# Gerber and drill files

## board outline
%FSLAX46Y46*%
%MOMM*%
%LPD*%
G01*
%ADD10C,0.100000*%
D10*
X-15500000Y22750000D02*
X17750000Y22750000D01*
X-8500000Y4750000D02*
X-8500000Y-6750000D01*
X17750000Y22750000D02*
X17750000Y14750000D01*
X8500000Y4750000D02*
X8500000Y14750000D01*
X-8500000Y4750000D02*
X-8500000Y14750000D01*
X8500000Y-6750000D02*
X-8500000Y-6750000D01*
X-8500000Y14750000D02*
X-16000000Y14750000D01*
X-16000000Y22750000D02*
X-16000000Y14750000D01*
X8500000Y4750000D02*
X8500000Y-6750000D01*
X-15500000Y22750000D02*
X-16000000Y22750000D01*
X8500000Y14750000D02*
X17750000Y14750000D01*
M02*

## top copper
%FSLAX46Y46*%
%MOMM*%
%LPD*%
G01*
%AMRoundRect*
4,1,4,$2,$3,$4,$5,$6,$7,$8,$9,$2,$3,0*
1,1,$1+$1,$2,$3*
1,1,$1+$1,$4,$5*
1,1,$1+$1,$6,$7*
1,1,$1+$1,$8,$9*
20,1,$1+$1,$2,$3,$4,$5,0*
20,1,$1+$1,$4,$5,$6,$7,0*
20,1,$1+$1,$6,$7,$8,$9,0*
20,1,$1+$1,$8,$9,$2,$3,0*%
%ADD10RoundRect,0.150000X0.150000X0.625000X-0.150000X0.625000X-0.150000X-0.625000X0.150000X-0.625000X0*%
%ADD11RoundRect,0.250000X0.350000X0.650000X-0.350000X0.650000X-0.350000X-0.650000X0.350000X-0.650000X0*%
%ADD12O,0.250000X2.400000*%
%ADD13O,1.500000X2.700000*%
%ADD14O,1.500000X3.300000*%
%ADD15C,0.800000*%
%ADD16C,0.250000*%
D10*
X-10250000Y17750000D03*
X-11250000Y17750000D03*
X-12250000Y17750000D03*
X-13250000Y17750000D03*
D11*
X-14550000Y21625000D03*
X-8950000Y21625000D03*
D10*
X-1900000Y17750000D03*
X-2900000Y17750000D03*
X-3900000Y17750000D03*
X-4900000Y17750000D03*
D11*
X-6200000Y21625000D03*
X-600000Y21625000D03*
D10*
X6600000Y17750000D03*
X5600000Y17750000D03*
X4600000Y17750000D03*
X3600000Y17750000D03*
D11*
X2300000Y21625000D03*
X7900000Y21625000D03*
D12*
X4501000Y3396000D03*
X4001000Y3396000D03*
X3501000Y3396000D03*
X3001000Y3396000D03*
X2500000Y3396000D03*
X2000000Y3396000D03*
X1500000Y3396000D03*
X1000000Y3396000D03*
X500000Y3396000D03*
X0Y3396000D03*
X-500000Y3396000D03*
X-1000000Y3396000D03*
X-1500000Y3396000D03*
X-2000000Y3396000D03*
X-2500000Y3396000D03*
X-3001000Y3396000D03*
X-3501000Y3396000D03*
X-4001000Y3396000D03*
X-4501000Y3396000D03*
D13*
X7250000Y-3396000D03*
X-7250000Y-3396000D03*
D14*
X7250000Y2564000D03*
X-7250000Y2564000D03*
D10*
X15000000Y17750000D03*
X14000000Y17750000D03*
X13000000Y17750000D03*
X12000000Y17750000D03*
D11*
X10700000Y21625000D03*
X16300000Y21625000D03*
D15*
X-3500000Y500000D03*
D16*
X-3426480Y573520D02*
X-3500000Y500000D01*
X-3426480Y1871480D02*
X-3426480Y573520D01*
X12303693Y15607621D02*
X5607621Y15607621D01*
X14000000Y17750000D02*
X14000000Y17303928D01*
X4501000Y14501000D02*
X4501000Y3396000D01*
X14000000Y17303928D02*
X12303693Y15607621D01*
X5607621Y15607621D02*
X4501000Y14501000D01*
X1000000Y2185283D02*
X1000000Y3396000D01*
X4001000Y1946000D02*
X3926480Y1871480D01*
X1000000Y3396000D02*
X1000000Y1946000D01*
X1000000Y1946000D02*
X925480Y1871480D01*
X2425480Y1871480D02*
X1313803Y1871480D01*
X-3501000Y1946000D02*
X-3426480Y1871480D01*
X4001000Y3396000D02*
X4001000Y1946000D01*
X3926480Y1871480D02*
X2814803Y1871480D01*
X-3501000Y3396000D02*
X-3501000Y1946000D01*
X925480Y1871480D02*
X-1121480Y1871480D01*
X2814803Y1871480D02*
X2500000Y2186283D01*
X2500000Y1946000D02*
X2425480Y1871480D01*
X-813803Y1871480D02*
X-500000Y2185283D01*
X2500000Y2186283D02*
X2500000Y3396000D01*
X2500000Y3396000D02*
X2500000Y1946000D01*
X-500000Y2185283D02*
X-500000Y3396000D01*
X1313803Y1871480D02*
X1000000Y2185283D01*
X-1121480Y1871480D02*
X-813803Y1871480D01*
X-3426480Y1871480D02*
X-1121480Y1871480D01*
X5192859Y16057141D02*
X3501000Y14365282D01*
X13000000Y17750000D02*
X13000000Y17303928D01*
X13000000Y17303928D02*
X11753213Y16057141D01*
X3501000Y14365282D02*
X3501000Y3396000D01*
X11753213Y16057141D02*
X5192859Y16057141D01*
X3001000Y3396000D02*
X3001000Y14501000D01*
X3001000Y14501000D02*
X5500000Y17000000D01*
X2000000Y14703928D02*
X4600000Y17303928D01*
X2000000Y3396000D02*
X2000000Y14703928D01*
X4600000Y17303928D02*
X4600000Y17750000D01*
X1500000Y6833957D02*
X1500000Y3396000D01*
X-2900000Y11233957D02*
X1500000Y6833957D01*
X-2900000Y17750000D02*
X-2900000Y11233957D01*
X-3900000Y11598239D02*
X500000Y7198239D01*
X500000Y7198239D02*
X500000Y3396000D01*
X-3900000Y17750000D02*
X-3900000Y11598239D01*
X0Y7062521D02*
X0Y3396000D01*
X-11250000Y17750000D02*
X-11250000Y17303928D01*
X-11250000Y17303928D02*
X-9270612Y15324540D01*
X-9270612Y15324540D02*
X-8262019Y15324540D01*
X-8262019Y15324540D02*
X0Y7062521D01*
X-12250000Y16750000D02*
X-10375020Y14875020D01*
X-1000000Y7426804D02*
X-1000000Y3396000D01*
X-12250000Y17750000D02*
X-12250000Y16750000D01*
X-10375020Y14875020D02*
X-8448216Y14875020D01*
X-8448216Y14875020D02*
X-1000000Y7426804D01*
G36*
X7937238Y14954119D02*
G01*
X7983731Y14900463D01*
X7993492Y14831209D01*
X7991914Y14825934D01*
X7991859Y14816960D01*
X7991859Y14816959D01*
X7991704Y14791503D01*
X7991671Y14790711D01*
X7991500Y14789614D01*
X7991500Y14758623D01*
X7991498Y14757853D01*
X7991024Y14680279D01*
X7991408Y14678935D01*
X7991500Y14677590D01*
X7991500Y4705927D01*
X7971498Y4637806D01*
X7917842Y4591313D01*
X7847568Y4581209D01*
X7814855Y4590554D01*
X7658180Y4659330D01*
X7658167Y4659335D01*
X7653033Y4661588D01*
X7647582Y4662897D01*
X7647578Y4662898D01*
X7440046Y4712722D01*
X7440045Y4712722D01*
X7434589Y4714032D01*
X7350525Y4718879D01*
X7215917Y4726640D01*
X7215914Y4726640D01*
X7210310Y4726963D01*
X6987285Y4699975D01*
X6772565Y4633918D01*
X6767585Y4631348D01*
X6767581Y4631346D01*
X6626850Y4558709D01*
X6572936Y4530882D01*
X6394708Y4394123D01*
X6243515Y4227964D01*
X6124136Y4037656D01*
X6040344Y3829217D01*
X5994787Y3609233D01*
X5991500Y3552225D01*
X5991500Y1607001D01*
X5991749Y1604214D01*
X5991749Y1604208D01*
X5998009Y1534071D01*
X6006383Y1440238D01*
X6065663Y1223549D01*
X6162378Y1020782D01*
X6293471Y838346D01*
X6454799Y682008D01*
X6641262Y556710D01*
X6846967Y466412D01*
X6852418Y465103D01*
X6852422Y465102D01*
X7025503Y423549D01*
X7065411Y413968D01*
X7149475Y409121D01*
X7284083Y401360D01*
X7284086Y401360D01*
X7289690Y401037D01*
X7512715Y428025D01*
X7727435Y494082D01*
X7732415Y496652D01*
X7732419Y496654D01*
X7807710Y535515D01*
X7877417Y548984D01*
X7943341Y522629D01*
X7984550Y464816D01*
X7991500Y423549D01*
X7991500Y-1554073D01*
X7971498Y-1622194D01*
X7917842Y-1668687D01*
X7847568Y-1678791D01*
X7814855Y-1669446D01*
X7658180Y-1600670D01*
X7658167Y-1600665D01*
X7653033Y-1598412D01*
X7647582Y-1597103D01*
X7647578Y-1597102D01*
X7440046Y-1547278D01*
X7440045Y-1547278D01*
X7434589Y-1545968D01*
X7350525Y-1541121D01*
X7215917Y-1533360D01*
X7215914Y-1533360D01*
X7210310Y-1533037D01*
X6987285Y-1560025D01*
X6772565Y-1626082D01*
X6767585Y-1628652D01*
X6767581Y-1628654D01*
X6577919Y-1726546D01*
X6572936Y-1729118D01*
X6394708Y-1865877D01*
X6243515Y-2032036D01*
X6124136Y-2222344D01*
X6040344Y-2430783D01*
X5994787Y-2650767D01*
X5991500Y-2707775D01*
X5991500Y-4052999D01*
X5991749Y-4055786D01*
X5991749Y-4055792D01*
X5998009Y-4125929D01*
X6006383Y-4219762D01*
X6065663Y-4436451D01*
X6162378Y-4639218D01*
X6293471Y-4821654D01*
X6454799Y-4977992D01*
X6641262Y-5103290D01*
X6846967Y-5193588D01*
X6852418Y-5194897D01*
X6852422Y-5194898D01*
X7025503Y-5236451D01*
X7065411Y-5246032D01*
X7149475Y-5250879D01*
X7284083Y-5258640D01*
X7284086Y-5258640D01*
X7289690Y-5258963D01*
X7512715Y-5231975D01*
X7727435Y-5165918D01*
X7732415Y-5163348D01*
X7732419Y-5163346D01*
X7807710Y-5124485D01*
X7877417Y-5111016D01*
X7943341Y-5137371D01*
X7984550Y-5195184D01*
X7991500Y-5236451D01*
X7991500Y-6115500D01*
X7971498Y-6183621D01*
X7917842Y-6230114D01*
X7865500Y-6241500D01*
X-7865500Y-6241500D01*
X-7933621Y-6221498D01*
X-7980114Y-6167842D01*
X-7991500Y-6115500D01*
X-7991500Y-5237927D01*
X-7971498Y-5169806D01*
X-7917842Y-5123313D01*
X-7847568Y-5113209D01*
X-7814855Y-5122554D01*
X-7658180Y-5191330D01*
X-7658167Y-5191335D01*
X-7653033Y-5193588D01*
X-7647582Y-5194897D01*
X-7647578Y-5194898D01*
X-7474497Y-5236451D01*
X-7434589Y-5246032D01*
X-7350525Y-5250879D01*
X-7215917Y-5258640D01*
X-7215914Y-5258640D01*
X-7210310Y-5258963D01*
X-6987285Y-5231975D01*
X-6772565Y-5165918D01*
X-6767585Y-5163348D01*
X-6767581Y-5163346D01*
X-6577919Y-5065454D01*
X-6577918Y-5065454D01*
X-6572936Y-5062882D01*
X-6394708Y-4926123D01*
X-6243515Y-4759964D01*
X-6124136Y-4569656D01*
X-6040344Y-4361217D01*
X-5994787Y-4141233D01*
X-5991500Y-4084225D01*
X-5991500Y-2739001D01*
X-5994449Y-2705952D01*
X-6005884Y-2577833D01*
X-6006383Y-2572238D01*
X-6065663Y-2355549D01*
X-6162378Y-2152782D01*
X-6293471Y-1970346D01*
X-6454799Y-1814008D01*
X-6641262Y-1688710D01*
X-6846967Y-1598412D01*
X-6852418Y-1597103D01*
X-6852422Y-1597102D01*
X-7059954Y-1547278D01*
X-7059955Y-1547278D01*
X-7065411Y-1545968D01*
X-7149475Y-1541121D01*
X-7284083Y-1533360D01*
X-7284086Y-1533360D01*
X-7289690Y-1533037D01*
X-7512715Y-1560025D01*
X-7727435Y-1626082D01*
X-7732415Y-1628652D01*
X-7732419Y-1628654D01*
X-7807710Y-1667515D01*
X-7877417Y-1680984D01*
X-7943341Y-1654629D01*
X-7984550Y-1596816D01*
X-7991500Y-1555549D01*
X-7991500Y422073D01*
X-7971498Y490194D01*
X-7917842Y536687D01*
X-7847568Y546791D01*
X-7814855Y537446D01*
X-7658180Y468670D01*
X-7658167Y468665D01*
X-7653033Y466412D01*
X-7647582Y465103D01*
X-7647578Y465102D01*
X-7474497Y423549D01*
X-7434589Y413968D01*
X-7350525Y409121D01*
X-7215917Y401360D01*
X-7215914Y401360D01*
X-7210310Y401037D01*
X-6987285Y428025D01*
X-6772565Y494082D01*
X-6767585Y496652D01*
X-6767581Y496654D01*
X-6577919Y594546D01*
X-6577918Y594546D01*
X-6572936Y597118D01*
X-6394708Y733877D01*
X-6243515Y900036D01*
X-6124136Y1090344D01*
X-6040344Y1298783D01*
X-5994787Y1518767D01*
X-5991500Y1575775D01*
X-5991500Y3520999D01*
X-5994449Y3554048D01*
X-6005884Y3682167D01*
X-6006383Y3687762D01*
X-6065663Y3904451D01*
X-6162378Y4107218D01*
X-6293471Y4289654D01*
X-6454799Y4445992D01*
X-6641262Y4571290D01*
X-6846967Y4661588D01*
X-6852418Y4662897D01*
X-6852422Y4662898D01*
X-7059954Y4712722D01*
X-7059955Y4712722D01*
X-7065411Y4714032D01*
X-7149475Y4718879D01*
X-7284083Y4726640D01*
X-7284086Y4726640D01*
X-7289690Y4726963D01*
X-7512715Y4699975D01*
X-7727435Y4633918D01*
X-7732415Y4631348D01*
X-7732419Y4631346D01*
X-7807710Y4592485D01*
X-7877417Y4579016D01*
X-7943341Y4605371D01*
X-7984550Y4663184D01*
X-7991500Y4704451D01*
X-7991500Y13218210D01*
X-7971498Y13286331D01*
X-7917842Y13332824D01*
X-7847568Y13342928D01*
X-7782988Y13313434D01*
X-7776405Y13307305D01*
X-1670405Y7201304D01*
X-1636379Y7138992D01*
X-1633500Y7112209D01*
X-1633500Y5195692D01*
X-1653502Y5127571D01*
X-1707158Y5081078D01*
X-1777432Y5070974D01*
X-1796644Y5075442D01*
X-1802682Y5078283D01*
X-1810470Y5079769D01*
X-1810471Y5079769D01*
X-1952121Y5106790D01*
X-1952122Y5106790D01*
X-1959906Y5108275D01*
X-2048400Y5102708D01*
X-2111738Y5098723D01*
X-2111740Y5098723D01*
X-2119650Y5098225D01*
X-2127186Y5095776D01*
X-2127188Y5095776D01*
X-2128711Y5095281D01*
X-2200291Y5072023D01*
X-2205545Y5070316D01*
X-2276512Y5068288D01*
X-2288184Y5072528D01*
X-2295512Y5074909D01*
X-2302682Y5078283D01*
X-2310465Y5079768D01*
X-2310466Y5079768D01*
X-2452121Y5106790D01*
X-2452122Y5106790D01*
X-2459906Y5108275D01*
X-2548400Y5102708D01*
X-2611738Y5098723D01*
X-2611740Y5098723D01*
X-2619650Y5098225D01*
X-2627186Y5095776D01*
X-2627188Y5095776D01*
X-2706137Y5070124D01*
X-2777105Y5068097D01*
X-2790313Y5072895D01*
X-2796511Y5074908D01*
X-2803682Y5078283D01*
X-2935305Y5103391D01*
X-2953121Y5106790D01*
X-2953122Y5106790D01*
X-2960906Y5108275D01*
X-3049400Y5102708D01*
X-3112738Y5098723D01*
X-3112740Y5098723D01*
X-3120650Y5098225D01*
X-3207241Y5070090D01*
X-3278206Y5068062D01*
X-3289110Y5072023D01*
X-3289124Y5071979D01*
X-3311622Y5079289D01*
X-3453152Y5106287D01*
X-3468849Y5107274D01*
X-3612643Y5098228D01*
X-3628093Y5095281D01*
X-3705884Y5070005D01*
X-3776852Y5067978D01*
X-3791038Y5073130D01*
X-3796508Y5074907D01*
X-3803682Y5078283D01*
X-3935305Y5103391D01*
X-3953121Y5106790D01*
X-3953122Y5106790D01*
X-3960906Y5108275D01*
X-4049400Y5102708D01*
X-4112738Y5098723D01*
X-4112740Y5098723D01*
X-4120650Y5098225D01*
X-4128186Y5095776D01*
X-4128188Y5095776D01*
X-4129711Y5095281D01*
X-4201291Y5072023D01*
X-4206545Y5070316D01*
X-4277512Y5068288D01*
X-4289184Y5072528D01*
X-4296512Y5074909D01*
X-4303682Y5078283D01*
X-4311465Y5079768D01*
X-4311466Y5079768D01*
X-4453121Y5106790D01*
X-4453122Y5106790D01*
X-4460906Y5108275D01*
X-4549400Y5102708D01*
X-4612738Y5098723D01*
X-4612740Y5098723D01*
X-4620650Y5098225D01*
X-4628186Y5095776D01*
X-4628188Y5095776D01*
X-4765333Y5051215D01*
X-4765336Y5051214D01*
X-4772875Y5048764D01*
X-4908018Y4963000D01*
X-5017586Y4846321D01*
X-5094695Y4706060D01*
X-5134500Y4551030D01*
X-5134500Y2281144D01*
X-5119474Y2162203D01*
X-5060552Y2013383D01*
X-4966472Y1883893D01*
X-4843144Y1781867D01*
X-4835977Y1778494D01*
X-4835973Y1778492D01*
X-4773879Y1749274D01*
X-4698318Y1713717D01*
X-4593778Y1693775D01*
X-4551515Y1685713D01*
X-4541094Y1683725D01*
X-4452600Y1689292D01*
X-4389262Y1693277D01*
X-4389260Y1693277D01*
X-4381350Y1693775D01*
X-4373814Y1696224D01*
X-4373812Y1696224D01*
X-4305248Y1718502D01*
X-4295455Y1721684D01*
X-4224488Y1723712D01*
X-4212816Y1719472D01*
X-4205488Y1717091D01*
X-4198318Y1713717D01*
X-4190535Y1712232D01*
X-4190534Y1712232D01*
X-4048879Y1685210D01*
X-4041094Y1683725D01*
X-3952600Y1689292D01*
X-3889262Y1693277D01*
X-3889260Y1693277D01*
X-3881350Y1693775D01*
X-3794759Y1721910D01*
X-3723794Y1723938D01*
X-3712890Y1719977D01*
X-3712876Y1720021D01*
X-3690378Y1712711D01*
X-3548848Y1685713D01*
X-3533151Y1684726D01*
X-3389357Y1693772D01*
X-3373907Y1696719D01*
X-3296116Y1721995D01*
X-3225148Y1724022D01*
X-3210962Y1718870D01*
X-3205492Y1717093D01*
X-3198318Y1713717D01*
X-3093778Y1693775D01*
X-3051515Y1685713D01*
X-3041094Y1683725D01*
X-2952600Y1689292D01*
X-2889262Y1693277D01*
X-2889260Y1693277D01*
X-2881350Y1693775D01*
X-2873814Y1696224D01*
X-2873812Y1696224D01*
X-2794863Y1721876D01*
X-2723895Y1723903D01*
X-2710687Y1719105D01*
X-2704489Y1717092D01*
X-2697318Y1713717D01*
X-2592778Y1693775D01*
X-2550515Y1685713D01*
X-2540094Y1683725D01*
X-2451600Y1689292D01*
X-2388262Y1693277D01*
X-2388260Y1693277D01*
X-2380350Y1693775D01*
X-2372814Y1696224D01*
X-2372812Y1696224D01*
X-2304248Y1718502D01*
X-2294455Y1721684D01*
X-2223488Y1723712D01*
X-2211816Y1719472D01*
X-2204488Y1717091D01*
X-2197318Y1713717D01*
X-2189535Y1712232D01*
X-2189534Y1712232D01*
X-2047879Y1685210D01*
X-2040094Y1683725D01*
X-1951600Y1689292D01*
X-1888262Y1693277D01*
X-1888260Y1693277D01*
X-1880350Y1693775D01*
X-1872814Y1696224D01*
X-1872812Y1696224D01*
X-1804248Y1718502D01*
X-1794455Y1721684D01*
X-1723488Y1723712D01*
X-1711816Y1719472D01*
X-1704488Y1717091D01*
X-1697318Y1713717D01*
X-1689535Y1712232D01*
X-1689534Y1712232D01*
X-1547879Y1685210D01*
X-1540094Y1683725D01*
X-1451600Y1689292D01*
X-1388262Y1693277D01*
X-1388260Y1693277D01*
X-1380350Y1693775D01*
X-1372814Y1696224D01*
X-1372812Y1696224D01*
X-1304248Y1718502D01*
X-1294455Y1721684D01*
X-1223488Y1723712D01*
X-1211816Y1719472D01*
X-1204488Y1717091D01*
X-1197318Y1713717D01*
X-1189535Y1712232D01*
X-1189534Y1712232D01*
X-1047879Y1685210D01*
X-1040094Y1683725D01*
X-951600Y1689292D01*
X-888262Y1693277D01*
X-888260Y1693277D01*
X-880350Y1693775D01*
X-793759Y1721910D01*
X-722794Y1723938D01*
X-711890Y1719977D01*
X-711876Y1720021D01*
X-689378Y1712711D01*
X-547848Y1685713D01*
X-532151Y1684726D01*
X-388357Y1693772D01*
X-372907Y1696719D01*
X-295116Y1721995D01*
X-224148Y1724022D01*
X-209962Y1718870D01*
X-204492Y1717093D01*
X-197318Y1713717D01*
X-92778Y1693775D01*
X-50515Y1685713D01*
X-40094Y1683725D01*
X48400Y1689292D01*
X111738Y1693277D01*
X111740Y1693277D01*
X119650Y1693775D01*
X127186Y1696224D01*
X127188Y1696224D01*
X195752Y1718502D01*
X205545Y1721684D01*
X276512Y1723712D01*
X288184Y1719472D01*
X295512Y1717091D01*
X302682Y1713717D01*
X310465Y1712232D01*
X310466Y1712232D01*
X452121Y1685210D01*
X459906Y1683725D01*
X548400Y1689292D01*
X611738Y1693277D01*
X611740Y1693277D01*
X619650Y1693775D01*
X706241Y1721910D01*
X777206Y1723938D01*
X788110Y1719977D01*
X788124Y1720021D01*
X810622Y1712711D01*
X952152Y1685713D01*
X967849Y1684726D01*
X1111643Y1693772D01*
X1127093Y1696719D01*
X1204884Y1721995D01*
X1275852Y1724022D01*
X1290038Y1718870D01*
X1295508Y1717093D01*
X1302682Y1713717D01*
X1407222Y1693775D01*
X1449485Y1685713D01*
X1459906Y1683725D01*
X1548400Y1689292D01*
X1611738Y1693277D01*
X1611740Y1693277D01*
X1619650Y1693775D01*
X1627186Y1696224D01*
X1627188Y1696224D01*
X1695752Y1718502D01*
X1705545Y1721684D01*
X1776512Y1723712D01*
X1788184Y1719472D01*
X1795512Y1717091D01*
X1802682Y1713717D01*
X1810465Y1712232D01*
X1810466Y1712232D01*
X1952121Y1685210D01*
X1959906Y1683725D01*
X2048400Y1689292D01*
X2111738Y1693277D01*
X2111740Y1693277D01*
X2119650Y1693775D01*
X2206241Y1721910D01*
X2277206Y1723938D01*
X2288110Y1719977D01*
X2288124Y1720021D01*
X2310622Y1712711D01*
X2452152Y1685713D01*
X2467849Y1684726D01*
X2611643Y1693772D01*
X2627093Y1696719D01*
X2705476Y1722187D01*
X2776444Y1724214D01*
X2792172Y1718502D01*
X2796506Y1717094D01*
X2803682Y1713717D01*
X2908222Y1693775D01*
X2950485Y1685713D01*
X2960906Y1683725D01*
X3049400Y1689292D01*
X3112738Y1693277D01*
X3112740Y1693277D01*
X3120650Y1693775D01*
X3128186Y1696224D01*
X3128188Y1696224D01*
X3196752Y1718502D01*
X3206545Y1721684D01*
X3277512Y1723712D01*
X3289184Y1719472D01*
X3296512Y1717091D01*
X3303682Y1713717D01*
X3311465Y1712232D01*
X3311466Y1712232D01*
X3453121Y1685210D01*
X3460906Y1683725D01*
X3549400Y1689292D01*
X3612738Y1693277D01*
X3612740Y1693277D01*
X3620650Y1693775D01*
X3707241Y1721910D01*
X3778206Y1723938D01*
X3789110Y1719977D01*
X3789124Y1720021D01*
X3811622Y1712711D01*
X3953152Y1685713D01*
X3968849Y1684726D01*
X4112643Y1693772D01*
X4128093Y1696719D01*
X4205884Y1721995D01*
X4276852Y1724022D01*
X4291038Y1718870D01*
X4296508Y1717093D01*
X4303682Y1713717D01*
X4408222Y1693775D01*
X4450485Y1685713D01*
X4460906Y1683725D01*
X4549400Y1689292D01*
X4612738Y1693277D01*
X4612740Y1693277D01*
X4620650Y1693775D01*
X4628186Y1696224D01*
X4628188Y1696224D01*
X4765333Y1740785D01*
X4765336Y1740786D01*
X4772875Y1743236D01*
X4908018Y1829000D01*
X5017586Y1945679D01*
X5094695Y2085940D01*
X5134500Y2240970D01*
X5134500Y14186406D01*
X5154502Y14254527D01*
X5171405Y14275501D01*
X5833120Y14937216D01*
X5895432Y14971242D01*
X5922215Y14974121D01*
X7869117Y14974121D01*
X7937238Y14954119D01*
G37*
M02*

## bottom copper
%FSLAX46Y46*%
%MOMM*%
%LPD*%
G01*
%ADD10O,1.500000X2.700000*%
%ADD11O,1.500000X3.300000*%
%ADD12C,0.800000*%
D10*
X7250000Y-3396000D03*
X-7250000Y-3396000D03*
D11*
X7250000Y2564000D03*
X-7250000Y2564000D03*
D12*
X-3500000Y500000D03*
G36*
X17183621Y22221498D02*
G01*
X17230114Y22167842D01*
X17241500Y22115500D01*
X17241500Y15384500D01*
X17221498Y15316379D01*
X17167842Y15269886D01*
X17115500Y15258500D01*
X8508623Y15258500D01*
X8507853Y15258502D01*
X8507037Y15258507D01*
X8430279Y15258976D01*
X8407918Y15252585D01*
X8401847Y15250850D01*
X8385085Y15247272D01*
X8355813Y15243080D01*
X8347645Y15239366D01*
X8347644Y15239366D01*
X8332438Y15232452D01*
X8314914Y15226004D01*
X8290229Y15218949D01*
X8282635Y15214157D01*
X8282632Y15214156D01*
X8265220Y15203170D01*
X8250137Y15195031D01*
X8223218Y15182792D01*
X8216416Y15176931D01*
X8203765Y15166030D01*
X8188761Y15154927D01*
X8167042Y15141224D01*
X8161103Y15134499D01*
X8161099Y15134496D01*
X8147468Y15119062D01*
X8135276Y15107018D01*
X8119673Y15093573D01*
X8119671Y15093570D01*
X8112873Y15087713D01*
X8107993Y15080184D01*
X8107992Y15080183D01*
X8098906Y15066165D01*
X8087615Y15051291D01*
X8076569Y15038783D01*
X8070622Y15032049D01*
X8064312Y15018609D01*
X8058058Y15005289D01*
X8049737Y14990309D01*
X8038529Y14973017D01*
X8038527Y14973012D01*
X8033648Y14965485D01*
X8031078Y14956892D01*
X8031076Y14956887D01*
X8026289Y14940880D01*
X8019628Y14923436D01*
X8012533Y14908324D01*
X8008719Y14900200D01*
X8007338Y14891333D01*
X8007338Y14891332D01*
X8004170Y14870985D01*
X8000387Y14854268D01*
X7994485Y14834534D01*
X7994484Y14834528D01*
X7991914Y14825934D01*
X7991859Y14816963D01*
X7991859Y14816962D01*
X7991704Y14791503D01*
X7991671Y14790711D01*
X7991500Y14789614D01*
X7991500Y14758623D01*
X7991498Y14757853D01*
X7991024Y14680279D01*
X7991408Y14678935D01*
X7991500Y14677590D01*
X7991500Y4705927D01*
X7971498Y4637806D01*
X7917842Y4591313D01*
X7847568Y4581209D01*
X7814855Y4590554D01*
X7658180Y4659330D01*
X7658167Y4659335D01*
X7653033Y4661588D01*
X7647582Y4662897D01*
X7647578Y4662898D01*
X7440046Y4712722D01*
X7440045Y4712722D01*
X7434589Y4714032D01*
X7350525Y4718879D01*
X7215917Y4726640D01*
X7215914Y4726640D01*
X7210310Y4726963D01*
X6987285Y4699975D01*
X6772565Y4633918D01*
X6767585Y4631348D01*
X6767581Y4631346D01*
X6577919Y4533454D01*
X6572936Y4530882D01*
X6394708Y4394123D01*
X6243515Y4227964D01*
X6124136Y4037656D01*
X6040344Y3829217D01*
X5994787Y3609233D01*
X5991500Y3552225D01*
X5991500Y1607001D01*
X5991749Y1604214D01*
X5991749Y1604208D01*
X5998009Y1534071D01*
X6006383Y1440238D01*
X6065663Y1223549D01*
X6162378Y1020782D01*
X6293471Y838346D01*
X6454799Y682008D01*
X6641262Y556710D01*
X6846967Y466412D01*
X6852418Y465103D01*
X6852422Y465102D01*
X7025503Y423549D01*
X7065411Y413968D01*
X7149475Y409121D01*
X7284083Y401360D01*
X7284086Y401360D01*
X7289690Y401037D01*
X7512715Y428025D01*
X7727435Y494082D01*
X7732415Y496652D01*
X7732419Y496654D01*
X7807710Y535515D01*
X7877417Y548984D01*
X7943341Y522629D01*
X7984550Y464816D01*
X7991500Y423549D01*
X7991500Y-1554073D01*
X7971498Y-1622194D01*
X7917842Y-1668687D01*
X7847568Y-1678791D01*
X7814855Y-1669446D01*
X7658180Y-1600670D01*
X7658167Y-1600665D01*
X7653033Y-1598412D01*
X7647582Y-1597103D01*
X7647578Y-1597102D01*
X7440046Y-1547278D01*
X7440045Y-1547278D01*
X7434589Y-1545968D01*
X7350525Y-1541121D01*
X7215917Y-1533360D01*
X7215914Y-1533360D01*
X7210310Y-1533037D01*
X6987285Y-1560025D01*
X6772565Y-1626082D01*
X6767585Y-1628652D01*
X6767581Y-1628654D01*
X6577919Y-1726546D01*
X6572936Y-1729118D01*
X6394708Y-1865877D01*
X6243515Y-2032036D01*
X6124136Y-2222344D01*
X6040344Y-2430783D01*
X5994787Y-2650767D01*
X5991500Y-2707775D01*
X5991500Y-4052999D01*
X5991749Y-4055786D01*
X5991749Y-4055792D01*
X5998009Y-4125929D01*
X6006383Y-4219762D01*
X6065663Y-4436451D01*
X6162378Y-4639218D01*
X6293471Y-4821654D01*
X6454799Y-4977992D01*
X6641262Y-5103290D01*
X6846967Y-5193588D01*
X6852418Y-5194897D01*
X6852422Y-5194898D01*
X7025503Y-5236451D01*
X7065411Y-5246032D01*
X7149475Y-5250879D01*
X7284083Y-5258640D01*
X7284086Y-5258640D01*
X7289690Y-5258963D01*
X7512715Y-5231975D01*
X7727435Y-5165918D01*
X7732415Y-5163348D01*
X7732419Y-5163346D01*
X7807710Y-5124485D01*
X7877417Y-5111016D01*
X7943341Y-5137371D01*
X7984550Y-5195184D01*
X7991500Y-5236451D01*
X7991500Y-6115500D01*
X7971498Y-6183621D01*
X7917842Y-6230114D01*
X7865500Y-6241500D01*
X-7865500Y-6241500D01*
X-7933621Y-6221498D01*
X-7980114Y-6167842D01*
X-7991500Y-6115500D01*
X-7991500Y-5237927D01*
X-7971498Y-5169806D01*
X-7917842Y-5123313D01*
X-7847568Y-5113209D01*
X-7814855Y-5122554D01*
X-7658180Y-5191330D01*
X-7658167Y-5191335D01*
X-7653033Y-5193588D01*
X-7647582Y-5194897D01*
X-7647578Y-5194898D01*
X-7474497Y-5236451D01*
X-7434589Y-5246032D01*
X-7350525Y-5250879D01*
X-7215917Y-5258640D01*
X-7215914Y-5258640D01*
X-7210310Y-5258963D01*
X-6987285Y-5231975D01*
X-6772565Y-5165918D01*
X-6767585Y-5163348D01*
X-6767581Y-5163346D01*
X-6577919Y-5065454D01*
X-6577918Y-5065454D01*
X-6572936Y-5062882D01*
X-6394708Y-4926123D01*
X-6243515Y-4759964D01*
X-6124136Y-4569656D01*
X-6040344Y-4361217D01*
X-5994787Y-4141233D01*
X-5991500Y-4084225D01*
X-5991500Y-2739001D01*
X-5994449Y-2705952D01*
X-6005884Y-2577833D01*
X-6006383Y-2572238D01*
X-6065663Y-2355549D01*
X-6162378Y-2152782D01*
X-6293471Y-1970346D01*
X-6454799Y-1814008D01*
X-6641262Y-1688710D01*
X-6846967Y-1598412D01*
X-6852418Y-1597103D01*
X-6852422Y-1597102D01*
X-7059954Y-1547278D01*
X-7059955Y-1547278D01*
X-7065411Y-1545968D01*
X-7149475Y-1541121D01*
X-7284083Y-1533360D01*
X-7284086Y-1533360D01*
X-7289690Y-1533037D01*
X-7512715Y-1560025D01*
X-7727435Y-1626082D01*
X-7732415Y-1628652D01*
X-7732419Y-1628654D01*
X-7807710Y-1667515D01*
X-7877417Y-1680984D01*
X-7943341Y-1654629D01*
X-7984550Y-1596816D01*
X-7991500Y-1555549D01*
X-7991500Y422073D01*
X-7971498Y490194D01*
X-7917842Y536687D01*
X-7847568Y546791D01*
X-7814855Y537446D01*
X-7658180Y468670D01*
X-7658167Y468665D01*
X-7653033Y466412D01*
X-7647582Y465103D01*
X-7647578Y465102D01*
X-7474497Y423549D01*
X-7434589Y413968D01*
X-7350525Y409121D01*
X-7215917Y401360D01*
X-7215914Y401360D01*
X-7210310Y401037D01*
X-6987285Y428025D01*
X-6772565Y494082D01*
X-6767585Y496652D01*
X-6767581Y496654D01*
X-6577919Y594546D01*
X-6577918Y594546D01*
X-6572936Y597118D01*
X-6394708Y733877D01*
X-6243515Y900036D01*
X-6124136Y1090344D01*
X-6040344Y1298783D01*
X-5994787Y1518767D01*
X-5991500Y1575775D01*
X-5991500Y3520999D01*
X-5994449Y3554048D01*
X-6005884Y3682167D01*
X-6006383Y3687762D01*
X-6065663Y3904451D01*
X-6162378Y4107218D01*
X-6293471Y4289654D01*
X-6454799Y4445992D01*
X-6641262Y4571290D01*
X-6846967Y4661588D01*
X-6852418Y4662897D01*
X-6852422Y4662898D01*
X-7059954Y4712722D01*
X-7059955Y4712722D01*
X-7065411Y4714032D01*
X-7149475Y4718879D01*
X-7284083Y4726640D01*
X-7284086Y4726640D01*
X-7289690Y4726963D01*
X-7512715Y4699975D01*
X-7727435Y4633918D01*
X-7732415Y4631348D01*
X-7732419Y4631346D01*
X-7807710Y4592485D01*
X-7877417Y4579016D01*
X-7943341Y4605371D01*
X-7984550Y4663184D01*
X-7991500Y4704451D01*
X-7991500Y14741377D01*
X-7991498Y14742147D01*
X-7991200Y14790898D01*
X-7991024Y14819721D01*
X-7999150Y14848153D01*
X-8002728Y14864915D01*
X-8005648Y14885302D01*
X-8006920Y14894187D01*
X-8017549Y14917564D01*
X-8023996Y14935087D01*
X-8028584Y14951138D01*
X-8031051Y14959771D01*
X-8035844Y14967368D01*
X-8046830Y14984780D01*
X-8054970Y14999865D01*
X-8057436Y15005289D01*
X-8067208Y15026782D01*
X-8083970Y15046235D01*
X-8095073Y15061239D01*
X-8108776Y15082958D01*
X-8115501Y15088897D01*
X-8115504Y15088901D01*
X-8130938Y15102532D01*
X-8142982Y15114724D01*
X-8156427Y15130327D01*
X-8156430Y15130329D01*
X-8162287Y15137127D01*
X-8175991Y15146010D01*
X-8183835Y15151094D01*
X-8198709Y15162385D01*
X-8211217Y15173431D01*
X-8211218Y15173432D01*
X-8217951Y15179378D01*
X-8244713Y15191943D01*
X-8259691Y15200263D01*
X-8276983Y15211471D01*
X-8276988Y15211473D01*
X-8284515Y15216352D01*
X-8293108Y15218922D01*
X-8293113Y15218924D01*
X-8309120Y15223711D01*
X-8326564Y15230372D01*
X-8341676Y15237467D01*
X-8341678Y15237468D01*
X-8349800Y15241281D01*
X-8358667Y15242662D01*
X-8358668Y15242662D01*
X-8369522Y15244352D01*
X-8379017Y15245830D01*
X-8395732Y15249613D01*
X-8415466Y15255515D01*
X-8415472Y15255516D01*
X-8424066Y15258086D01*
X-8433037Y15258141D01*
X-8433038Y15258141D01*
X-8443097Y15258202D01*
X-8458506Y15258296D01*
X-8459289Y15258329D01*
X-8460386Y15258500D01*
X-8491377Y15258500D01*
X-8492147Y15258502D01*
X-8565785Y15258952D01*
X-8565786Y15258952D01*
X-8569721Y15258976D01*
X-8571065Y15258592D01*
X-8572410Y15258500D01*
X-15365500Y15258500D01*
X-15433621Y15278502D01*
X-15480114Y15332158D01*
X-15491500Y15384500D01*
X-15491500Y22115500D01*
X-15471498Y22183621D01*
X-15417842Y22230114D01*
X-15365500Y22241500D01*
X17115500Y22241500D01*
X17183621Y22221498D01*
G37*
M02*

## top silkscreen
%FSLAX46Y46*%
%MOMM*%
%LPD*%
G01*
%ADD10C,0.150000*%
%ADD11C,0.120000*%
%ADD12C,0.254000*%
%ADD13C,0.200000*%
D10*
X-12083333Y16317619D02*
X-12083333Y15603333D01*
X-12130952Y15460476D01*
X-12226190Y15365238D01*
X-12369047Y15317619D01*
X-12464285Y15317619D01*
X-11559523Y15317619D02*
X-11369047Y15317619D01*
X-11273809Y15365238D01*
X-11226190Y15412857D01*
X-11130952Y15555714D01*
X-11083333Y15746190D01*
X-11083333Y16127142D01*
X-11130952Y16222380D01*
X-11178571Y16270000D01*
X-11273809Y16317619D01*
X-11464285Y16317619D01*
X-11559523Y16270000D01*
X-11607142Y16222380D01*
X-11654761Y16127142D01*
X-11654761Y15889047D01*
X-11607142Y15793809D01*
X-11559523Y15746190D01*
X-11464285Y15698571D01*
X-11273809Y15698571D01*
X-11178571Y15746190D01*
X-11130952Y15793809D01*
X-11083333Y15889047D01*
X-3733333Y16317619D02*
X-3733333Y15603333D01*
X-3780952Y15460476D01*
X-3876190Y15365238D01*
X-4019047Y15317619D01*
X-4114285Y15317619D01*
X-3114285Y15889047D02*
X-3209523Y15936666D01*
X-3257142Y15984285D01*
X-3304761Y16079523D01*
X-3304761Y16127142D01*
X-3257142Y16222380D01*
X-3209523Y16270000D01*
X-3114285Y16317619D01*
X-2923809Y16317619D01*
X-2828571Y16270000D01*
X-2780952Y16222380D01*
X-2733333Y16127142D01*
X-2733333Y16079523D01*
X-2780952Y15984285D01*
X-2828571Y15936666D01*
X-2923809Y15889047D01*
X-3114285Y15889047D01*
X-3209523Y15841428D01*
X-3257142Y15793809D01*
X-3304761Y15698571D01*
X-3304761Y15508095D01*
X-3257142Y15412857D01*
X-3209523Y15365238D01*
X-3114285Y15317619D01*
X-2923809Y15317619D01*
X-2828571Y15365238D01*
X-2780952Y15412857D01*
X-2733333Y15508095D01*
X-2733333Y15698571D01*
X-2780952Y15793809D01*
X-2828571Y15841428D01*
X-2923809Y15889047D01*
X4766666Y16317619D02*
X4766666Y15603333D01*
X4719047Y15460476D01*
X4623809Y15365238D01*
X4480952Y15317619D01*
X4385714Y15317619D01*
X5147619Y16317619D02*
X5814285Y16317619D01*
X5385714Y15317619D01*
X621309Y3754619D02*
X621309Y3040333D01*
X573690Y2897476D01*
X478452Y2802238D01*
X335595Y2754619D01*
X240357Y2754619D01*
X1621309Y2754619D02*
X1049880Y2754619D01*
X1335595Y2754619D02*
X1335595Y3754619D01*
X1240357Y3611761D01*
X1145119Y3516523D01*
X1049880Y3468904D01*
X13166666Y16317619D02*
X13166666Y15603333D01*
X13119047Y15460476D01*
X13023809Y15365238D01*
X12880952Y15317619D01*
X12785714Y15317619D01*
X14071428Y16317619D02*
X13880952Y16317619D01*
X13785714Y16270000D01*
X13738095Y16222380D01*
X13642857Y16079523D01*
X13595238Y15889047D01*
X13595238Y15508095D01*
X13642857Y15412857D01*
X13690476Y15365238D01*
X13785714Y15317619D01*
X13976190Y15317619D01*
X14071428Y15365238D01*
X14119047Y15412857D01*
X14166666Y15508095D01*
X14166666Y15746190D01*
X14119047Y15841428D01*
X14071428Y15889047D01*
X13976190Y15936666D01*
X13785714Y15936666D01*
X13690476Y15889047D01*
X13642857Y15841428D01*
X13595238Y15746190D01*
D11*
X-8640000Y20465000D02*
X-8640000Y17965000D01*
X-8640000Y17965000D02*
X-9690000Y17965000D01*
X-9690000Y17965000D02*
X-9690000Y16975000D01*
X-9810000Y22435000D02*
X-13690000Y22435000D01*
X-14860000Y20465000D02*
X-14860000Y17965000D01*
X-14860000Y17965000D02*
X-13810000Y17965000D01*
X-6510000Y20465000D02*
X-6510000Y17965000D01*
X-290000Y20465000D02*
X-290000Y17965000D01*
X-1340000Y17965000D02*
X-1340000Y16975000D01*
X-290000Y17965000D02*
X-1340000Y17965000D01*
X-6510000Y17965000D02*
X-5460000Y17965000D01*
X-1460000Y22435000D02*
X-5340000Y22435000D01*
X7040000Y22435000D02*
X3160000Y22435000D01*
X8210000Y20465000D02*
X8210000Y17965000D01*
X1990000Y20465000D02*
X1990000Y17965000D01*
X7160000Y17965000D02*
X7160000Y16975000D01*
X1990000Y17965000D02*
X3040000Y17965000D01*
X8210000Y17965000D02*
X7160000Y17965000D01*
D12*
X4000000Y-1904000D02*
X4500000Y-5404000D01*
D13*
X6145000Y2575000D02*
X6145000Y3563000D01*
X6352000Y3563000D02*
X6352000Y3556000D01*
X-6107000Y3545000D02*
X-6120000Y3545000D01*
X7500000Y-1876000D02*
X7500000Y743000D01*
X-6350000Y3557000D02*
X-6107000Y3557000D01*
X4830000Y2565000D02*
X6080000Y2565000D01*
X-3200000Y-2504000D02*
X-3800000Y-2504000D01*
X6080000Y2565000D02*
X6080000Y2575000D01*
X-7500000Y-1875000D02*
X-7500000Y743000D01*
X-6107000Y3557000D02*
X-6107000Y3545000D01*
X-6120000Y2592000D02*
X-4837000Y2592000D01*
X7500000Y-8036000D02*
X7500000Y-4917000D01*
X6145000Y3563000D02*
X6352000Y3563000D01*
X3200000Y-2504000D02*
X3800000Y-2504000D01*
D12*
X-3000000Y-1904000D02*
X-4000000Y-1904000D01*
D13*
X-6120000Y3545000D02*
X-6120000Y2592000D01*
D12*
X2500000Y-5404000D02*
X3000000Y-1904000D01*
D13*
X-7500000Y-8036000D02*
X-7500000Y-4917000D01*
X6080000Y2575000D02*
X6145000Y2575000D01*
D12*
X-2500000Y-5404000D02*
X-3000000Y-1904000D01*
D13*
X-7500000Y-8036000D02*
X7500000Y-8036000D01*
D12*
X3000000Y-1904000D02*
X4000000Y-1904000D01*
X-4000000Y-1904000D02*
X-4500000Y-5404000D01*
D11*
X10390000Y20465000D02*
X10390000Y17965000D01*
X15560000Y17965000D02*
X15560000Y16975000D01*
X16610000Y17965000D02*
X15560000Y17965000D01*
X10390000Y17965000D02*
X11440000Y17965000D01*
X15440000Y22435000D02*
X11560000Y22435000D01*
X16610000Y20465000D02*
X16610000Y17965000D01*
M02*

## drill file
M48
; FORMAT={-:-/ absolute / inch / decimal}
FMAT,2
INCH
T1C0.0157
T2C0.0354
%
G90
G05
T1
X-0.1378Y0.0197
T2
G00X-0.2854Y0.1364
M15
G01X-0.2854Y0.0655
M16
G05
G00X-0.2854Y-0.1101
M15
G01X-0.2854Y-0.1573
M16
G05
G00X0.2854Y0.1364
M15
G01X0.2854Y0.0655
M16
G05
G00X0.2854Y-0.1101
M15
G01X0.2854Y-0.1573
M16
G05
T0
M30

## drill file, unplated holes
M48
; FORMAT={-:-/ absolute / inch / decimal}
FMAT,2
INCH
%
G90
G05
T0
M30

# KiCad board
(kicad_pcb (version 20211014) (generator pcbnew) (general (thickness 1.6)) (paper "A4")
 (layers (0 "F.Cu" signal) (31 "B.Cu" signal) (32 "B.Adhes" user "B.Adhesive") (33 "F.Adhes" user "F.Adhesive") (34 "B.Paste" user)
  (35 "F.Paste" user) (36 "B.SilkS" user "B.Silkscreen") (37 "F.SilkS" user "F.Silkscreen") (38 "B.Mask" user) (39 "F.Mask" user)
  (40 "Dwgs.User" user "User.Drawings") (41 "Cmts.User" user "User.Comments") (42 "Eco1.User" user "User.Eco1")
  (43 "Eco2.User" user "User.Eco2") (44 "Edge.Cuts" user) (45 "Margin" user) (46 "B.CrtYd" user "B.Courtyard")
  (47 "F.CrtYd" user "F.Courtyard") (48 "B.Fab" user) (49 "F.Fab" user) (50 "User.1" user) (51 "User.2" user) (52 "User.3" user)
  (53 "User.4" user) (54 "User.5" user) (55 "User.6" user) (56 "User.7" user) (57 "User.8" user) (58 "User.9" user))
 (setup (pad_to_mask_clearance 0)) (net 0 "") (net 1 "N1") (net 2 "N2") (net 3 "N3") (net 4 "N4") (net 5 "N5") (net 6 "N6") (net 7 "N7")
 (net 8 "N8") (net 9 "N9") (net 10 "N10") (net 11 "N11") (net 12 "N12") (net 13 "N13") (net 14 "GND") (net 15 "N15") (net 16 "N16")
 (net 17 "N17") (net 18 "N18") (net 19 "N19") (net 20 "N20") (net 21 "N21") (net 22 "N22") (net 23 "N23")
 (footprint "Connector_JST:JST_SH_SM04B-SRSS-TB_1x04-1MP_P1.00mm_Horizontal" (layer "F.Cu") (at -11.75 -19.75 180)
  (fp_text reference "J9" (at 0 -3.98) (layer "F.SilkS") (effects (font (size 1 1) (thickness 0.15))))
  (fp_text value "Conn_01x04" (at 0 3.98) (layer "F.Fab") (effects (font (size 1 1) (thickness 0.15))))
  (fp_line (start -3.11 0.715) (end -3.11 -1.785) (layer "F.SilkS") (width 0.12))
  (fp_line (start -3.11 -1.785) (end -2.06 -1.785) (layer "F.SilkS") (width 0.12))
  (fp_line (start -2.06 -1.785) (end -2.06 -2.775) (layer "F.SilkS") (width 0.12))
  (fp_line (start -1.94 2.685) (end 1.94 2.685) (layer "F.SilkS") (width 0.12))
  (fp_line (start 3.11 0.715) (end 3.11 -1.785) (layer "F.SilkS") (width 0.12))
  (fp_line (start 3.11 -1.785) (end 2.06 -1.785) (layer "F.SilkS") (width 0.12))
  (pad "1" smd roundrect (at -1.5 -2 180) (size 0.6 1.55) (layers "F.Cu" "F.Paste" "F.Mask") (roundrect_rratio 0.25) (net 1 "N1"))
  (pad "2" smd roundrect (at -0.5 -2 180) (size 0.6 1.55) (layers "F.Cu" "F.Paste" "F.Mask") (roundrect_rratio 0.25) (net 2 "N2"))
  (pad "3" smd roundrect (at 0.5 -2 180) (size 0.6 1.55) (layers "F.Cu" "F.Paste" "F.Mask") (roundrect_rratio 0.25) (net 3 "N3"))
  (pad "4" smd roundrect (at 1.5 -2 180) (size 0.6 1.55) (layers "F.Cu" "F.Paste" "F.Mask") (roundrect_rratio 0.25) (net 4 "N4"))
  (pad "MP" smd roundrect (at 2.8 1.875 180) (size 1.2 1.8) (layers "F.Cu" "F.Paste" "F.Mask") (roundrect_rratio 0.2083333333))
  (pad "MP" smd roundrect (at -2.8 1.875 180) (size 1.2 1.8) (layers "F.Cu" "F.Paste" "F.Mask") (roundrect_rratio 0.2083333333)))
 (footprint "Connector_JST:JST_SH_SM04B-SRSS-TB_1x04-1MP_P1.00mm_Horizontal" (layer "F.Cu") (at -3.4 -19.75 180)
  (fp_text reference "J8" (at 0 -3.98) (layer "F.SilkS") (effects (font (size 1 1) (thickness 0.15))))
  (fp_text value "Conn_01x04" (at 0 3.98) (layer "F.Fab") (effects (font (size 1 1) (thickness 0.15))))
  (fp_line (start 3.11 0.715) (end 3.11 -1.785) (layer "F.SilkS") (width 0.12))
  (fp_line (start -3.11 0.715) (end -3.11 -1.785) (layer "F.SilkS") (width 0.12))
  (fp_line (start -2.06 -1.785) (end -2.06 -2.775) (layer "F.SilkS") (width 0.12))
  (fp_line (start -3.11 -1.785) (end -2.06 -1.785) (layer "F.SilkS") (width 0.12))
  (fp_line (start 3.11 -1.785) (end 2.06 -1.785) (layer "F.SilkS") (width 0.12))
  (fp_line (start -1.94 2.685) (end 1.94 2.685) (layer "F.SilkS") (width 0.12))
  (pad "1" smd roundrect (at -1.5 -2 180) (size 0.6 1.55) (layers "F.Cu" "F.Paste" "F.Mask") (roundrect_rratio 0.25) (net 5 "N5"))
  (pad "2" smd roundrect (at -0.5 -2 180) (size 0.6 1.55) (layers "F.Cu" "F.Paste" "F.Mask") (roundrect_rratio 0.25) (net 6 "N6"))
  (pad "3" smd roundrect (at 0.5 -2 180) (size 0.6 1.55) (layers "F.Cu" "F.Paste" "F.Mask") (roundrect_rratio 0.25) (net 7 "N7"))
  (pad "4" smd roundrect (at 1.5 -2 180) (size 0.6 1.55) (layers "F.Cu" "F.Paste" "F.Mask") (roundrect_rratio 0.25) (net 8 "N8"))
  (pad "MP" smd roundrect (at 2.8 1.875 180) (size 1.2 1.8) (layers "F.Cu" "F.Paste" "F.Mask") (roundrect_rratio 0.2083333333))
  (pad "MP" smd roundrect (at -2.8 1.875 180) (size 1.2 1.8) (layers "F.Cu" "F.Paste" "F.Mask") (roundrect_rratio 0.2083333333)))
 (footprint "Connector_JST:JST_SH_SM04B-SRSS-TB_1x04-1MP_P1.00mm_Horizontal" (layer "F.Cu") (at 5.1 -19.75 180)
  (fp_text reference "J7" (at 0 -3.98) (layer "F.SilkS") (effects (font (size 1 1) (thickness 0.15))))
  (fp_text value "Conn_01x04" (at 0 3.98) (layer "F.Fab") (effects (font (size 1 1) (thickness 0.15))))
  (fp_line (start -1.94 2.685) (end 1.94 2.685) (layer "F.SilkS") (width 0.12))
  (fp_line (start -3.11 0.715) (end -3.11 -1.785) (layer "F.SilkS") (width 0.12))
  (fp_line (start 3.11 0.715) (end 3.11 -1.785) (layer "F.SilkS") (width 0.12))
  (fp_line (start -2.06 -1.785) (end -2.06 -2.775) (layer "F.SilkS") (width 0.12))
  (fp_line (start 3.11 -1.785) (end 2.06 -1.785) (layer "F.SilkS") (width 0.12))
  (fp_line (start -3.11 -1.785) (end -2.06 -1.785) (layer "F.SilkS") (width 0.12))
  (pad "1" smd roundrect (at -1.5 -2 180) (size 0.6 1.55) (layers "F.Cu" "F.Paste" "F.Mask") (roundrect_rratio 0.25) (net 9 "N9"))
  (pad "2" smd roundrect (at -0.5 -2 180) (size 0.6 1.55) (layers "F.Cu" "F.Paste" "F.Mask") (roundrect_rratio 0.25) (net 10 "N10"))
  (pad "3" smd roundrect (at 0.5 -2 180) (size 0.6 1.55) (layers "F.Cu" "F.Paste" "F.Mask") (roundrect_rratio 0.25) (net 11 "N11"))
  (pad "4" smd roundrect (at 1.5 -2 180) (size 0.6 1.55) (layers "F.Cu" "F.Paste" "F.Mask") (roundrect_rratio 0.25) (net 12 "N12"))
  (pad "MP" smd roundrect (at 2.8 1.875 180) (size 1.2 1.8) (layers "F.Cu" "F.Paste" "F.Mask") (roundrect_rratio 0.2083333333))
  (pad "MP" smd roundrect (at -2.8 1.875 180) (size 1.2 1.8) (layers "F.Cu" "F.Paste" "F.Mask") (roundrect_rratio 0.2083333333)))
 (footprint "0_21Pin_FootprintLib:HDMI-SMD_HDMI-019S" (layer "F.Cu") (at 0 0)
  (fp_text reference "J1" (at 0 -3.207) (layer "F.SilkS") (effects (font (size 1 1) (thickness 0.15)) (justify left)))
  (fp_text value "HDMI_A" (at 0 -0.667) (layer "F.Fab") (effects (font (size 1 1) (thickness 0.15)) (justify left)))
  (fp_line (start 4 1.904) (end 4.5 5.404) (layer "F.SilkS") (width 0.254))
  (fp_line (start 6.145 -2.575) (end 6.145 -3.563) (layer "F.SilkS") (width 0.2))
  (fp_line (start 6.352 -3.563) (end 6.352 -3.556) (layer "F.SilkS") (width 0.2))
  (fp_line (start -6.107 -3.545) (end -6.12 -3.545) (layer "F.SilkS") (width 0.2))
  (fp_line (start 7.5 1.876) (end 7.5 -0.743) (layer "F.SilkS") (width 0.2))
  (fp_line (start -6.35 -3.557) (end -6.107 -3.557) (layer "F.SilkS") (width 0.2))
  (fp_line (start 4.83 -2.565) (end 6.08 -2.565) (layer "F.SilkS") (width 0.2))
  (fp_line (start -3.2 2.504) (end -3.8 2.504) (layer "F.SilkS") (width 0.2))
  (fp_line (start 6.08 -2.565) (end 6.08 -2.575) (layer "F.SilkS") (width 0.2))
  (fp_line (start -7.5 1.875) (end -7.5 -0.743) (layer "F.SilkS") (width 0.2))
  (fp_line (start -6.107 -3.557) (end -6.107 -3.545) (layer "F.SilkS") (width 0.2))
  (fp_line (start -6.12 -2.592) (end -4.837 -2.592) (layer "F.SilkS") (width 0.2))
  (fp_line (start 7.5 8.036) (end 7.5 4.917) (layer "F.SilkS") (width 0.2))
  (fp_line (start 6.145 -3.563) (end 6.352 -3.563) (layer "F.SilkS") (width 0.2))
  (fp_line (start 3.2 2.504) (end 3.8 2.504) (layer "F.SilkS") (width 0.2))
  (fp_line (start -3 1.904) (end -4 1.904) (layer "F.SilkS") (width 0.254))
  (fp_line (start -6.12 -3.545) (end -6.12 -2.592) (layer "F.SilkS") (width 0.2))
  (fp_line (start 2.5 5.404) (end 3 1.904) (layer "F.SilkS") (width 0.254))
  (fp_line (start -7.5 8.036) (end -7.5 4.917) (layer "F.SilkS") (width 0.2))
  (fp_line (start 6.08 -2.575) (end 6.145 -2.575) (layer "F.SilkS") (width 0.2))
  (fp_line (start -2.5 5.404) (end -3 1.904) (layer "F.SilkS") (width 0.254))
  (fp_line (start -7.5 8.036) (end 7.5 8.036) (layer "F.SilkS") (width 0.2))
  (fp_line (start 3 1.904) (end 4 1.904) (layer "F.SilkS") (width 0.254))
  (fp_line (start -4 1.904) (end -4.5 5.404) (layer "F.SilkS") (width 0.254))
  (pad "1" smd oval (at 4.501 -3.396) (size 0.25 2.4) (layers "F.Cu" "F.Paste" "F.Mask") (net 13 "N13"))
  (pad "2" smd oval (at 4.001 -3.396) (size 0.25 2.4) (layers "F.Cu" "F.Paste" "F.Mask") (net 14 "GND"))
  (pad "3" smd oval (at 3.501 -3.396) (size 0.25 2.4) (layers "F.Cu" "F.Paste" "F.Mask") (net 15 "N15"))
  (pad "4" smd oval (at 3.001 -3.396) (size 0.25 2.4) (layers "F.Cu" "F.Paste" "F.Mask") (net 10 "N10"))
  (pad "5" smd oval (at 2.5 -3.396) (size 0.25 2.4) (layers "F.Cu" "F.Paste" "F.Mask") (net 14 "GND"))
  (pad "6" smd oval (at 2 -3.396) (size 0.25 2.4) (layers "F.Cu" "F.Paste" "F.Mask") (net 11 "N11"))
  (pad "7" smd oval (at 1.5 -3.396) (size 0.25 2.4) (layers "F.Cu" "F.Paste" "F.Mask") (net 6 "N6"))
  (pad "8" smd oval (at 1 -3.396) (size 0.25 2.4) (layers "F.Cu" "F.Paste" "F.Mask") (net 14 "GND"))
  (pad "9" smd oval (at 0.5 -3.396) (size 0.25 2.4) (layers "F.Cu" "F.Paste" "F.Mask") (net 7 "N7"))
  (pad "10" smd oval (at 0 -3.396) (size 0.25 2.4) (layers "F.Cu" "F.Paste" "F.Mask") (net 2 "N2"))
  (pad "11" smd oval (at -0.5 -3.396) (size 0.25 2.4) (layers "F.Cu" "F.Paste" "F.Mask") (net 14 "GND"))
  (pad "12" smd oval (at -1 -3.396) (size 0.25 2.4) (layers "F.Cu" "F.Paste" "F.Mask") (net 3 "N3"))
  (pad "13" smd oval (at -1.5 -3.396) (size 0.25 2.4) (layers "F.Cu" "F.Paste" "F.Mask") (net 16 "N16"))
  (pad "14" smd oval (at -2 -3.396) (size 0.25 2.4) (layers "F.Cu" "F.Paste" "F.Mask") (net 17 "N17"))
  (pad "15" smd oval (at -2.5 -3.396) (size 0.25 2.4) (layers "F.Cu" "F.Paste" "F.Mask") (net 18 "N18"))
  (pad "16" smd oval (at -3.001 -3.396) (size 0.25 2.4) (layers "F.Cu" "F.Paste" "F.Mask") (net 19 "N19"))
  (pad "17" smd oval (at -3.501 -3.396) (size 0.25 2.4) (layers "F.Cu" "F.Paste" "F.Mask") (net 14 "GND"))
  (pad "18" smd oval (at -4.001 -3.396) (size 0.25 2.4) (layers "F.Cu" "F.Paste" "F.Mask") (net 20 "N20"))
  (pad "19" smd oval (at -4.501 -3.396) (size 0.25 2.4) (layers "F.Cu" "F.Paste" "F.Mask") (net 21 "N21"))
  (pad "20" thru_hole oval (at 7.25 3.396) (size 1.5 2.7) (drill oval 0.9 2.1) (layers *.Cu *.Mask))
  (pad "21" thru_hole oval (at -7.25 3.396) (size 1.5 2.7) (drill oval 0.9 2.1) (layers *.Cu *.Mask))
  (pad "22" thru_hole oval (at 7.25 -2.564) (size 1.5 3.3) (drill oval 0.9 2.7) (layers *.Cu *.Mask))
  (pad "23" thru_hole oval (at -7.25 -2.564) (size 1.5 3.3) (drill oval 0.9 2.7) (layers *.Cu *.Mask)))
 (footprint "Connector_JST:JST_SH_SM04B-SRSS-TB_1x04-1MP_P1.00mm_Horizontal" (layer "F.Cu") (at 13.5 -19.75 180)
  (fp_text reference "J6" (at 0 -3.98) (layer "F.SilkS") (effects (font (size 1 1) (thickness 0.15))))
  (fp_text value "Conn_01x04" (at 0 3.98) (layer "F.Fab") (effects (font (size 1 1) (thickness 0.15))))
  (fp_line (start 3.11 0.715) (end 3.11 -1.785) (layer "F.SilkS") (width 0.12))
  (fp_line (start -2.06 -1.785) (end -2.06 -2.775) (layer "F.SilkS") (width 0.12))
  (fp_line (start -3.11 -1.785) (end -2.06 -1.785) (layer "F.SilkS") (width 0.12))
  (fp_line (start 3.11 -1.785) (end 2.06 -1.785) (layer "F.SilkS") (width 0.12))
  (fp_line (start -1.94 2.685) (end 1.94 2.685) (layer "F.SilkS") (width 0.12))
  (fp_line (start -3.11 0.715) (end -3.11 -1.785) (layer "F.SilkS") (width 0.12))
  (pad "1" smd roundrect (at -1.5 -2 180) (size 0.6 1.55) (layers "F.Cu" "F.Paste" "F.Mask") (roundrect_rratio 0.25) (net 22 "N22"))
  (pad "2" smd roundrect (at -0.5 -2 180) (size 0.6 1.55) (layers "F.Cu" "F.Paste" "F.Mask") (roundrect_rratio 0.25) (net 13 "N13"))
  (pad "3" smd roundrect (at 0.5 -2 180) (size 0.6 1.55) (layers "F.Cu" "F.Paste" "F.Mask") (roundrect_rratio 0.25) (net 15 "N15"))
  (pad "4" smd roundrect (at 1.5 -2 180) (size 0.6 1.55) (layers "F.Cu" "F.Paste" "F.Mask") (roundrect_rratio 0.25) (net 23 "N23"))
  (pad "MP" smd roundrect (at 2.8 1.875 180) (size 1.2 1.8) (layers "F.Cu" "F.Paste" "F.Mask") (roundrect_rratio 0.2083333333))
  (pad "MP" smd roundrect (at -2.8 1.875 180) (size 1.2 1.8) (layers "F.Cu" "F.Paste" "F.Mask") (roundrect_rratio 0.2083333333)))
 (gr_line (start -15.5 -22.75) (end 17.75 -22.75) (layer "Edge.Cuts") (width 0.1))
 (gr_line (start -8.5 -4.75) (end -8.5 6.75) (layer "Edge.Cuts") (width 0.1))
 (gr_line (start 17.75 -22.75) (end 17.75 -14.75) (layer "Edge.Cuts") (width 0.1))
 (gr_line (start 8.5 -4.75) (end 8.5 -14.75) (layer "Edge.Cuts") (width 0.1))
 (gr_line (start -8.5 -4.75) (end -8.5 -14.75) (layer "Edge.Cuts") (width 0.1))
 (gr_line (start 8.5 6.75) (end -8.5 6.75) (layer "Edge.Cuts") (width 0.1))
 (gr_line (start -8.5 -14.75) (end -16 -14.75) (layer "Edge.Cuts") (width 0.1))
 (gr_line (start -16 -22.75) (end -16 -14.75) (layer "Edge.Cuts") (width 0.1))
 (gr_line (start 8.5 -4.75) (end 8.5 6.75) (layer "Edge.Cuts") (width 0.1))
 (gr_line (start -15.5 -22.75) (end -16 -22.75) (layer "Edge.Cuts") (width 0.1))
 (gr_line (start 8.5 -14.75) (end 17.75 -14.75) (layer "Edge.Cuts") (width 0.1))
 (segment (start 12.303693 -15.607621) (end 5.607621 -15.607621) (width 0.25) (layer "F.Cu") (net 13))
 (segment (start 14 -17.75) (end 14 -17.303928) (width 0.25) (layer "F.Cu") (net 13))
 (segment (start 4.501 -14.501) (end 4.501 -3.396) (width 0.25) (layer "F.Cu") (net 13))
 (segment (start 14 -17.303928) (end 12.303693 -15.607621) (width 0.25) (layer "F.Cu") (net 13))
 (segment (start 5.607621 -15.607621) (end 4.501 -14.501) (width 0.25) (layer "F.Cu") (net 13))
 (segment (start -3.42648 -1.87148) (end -3.42648 -0.57352) (width 0.25) (layer "F.Cu") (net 14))
 (segment (start 1 -2.185283) (end 1 -3.396) (width 0.25) (layer "F.Cu") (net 14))
 (segment (start 4.001 -1.946) (end 3.92648 -1.87148) (width 0.25) (layer "F.Cu") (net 14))
 (segment (start 1 -3.396) (end 1 -1.946) (width 0.25) (layer "F.Cu") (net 14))
 (segment (start 1 -1.946) (end 0.92548 -1.87148) (width 0.25) (layer "F.Cu") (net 14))
 (segment (start 2.42548 -1.87148) (end 1.313803 -1.87148) (width 0.25) (layer "F.Cu") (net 14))
 (segment (start -3.501 -1.946) (end -3.42648 -1.87148) (width 0.25) (layer "F.Cu") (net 14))
 (segment (start 4.001 -3.396) (end 4.001 -1.946) (width 0.25) (layer "F.Cu") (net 14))
 (segment (start 3.92648 -1.87148) (end 2.814803 -1.87148) (width 0.25) (layer "F.Cu") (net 14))
 (segment (start -3.501 -3.396) (end -3.501 -1.946) (width 0.25) (layer "F.Cu") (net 14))
 (segment (start 0.92548 -1.87148) (end -1.12148 -1.87148) (width 0.25) (layer "F.Cu") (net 14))
 (segment (start 2.814803 -1.87148) (end 2.5 -2.186283) (width 0.25) (layer "F.Cu") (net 14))
 (segment (start 2.5 -1.946) (end 2.42548 -1.87148) (width 0.25) (layer "F.Cu") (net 14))
 (segment (start -0.813803 -1.87148) (end -0.5 -2.185283) (width 0.25) (layer "F.Cu") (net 14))
 (segment (start -3.42648 -0.57352) (end -3.5 -0.5) (width 0.25) (layer "F.Cu") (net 14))
 (segment (start 2.5 -2.186283) (end 2.5 -3.396) (width 0.25) (layer "F.Cu") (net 14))
 (segment (start 2.5 -3.396) (end 2.5 -1.946) (width 0.25) (layer "F.Cu") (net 14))
 (segment (start -0.5 -2.185283) (end -0.5 -3.396) (width 0.25) (layer "F.Cu") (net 14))
 (segment (start 1.313803 -1.87148) (end 1 -2.185283) (width 0.25) (layer "F.Cu") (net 14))
 (segment (start -1.12148 -1.87148) (end -0.813803 -1.87148) (width 0.25) (layer "F.Cu") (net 14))
 (segment (start -3.42648 -1.87148) (end -1.12148 -1.87148) (width 0.25) (layer "F.Cu") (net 14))
 (via (at -3.5 -0.5) (size 0.8) (drill 0.4) (layers "F.Cu" "B.Cu") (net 14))
 (segment (start 5.192859 -16.057141) (end 3.501 -14.365282) (width 0.25) (layer "F.Cu") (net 15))
 (segment (start 13 -17.75) (end 13 -17.303928) (width 0.25) (layer "F.Cu") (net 15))
 (segment (start 13 -17.303928) (end 11.753213 -16.057141) (width 0.25) (layer "F.Cu") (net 15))
 (segment (start 3.501 -14.365282) (end 3.501 -3.396) (width 0.25) (layer "F.Cu") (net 15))
 (segment (start 11.753213 -16.057141) (end 5.192859 -16.057141) (width 0.25) (layer "F.Cu") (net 15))
 (segment (start 3.001 -3.396) (end 3.001 -14.501) (width 0.25) (layer "F.Cu") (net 10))
 (segment (start 3.001 -14.501) (end 5.5 -17) (width 0.25) (layer "F.Cu") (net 10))
 (segment (start 2 -14.703928) (end 4.6 -17.303928) (width 0.25) (layer "F.Cu") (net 11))
 (segment (start 2 -3.396) (end 2 -14.703928) (width 0.25) (layer "F.Cu") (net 11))
 (segment (start 4.6 -17.303928) (end 4.6 -17.75) (width 0.25) (layer "F.Cu") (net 11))
 (segment (start 1.5 -6.833957) (end 1.5 -3.396) (width 0.25) (layer "F.Cu") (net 6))
 (segment (start -2.9 -11.233957) (end 1.5 -6.833957) (width 0.25) (layer "F.Cu") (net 6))
 (segment (start -2.9 -17.75) (end -2.9 -11.233957) (width 0.25) (layer "F.Cu") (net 6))
 (segment (start -3.9 -11.598239) (end 0.5 -7.198239) (width 0.25) (layer "F.Cu") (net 7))
 (segment (start 0.5 -7.198239) (end 0.5 -3.396) (width 0.25) (layer "F.Cu") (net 7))
 (segment (start -3.9 -17.75) (end -3.9 -11.598239) (width 0.25) (layer "F.Cu") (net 7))
 (segment (start 0 -7.062521) (end 0 -3.396) (width 0.25) (layer "F.Cu") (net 2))
 (segment (start -11.25 -17.75) (end -11.25 -17.303928) (width 0.25) (layer "F.Cu") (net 2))
 (segment (start -11.25 -17.303928) (end -9.270612 -15.32454) (width 0.25) (layer "F.Cu") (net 2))
 (segment (start -9.270612 -15.32454) (end -8.262019 -15.32454) (width 0.25) (layer "F.Cu") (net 2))
 (segment (start -8.262019 -15.32454) (end 0 -7.062521) (width 0.25) (layer "F.Cu") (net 2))
 (segment (start -12.25 -16.75) (end -10.37502 -14.87502) (width 0.25) (layer "F.Cu") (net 3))
 (segment (start -1 -7.426804) (end -1 -3.396) (width 0.25) (layer "F.Cu") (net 3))
 (segment (start -12.25 -17.75) (end -12.25 -16.75) (width 0.25) (layer "F.Cu") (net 3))
 (segment (start -10.37502 -14.87502) (end -8.448216 -14.87502) (width 0.25) (layer "F.Cu") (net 3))
 (segment (start -8.448216 -14.87502) (end -1 -7.426804) (width 0.25) (layer "F.Cu") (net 3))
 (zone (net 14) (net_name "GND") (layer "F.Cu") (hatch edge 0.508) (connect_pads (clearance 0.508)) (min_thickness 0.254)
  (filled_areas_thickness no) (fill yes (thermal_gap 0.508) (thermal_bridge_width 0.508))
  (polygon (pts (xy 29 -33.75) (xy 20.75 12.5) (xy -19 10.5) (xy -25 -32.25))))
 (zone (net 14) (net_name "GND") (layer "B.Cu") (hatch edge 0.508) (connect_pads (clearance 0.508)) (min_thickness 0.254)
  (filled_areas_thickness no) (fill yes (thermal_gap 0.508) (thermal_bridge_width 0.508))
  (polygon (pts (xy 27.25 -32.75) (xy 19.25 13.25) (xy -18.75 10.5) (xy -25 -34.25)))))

